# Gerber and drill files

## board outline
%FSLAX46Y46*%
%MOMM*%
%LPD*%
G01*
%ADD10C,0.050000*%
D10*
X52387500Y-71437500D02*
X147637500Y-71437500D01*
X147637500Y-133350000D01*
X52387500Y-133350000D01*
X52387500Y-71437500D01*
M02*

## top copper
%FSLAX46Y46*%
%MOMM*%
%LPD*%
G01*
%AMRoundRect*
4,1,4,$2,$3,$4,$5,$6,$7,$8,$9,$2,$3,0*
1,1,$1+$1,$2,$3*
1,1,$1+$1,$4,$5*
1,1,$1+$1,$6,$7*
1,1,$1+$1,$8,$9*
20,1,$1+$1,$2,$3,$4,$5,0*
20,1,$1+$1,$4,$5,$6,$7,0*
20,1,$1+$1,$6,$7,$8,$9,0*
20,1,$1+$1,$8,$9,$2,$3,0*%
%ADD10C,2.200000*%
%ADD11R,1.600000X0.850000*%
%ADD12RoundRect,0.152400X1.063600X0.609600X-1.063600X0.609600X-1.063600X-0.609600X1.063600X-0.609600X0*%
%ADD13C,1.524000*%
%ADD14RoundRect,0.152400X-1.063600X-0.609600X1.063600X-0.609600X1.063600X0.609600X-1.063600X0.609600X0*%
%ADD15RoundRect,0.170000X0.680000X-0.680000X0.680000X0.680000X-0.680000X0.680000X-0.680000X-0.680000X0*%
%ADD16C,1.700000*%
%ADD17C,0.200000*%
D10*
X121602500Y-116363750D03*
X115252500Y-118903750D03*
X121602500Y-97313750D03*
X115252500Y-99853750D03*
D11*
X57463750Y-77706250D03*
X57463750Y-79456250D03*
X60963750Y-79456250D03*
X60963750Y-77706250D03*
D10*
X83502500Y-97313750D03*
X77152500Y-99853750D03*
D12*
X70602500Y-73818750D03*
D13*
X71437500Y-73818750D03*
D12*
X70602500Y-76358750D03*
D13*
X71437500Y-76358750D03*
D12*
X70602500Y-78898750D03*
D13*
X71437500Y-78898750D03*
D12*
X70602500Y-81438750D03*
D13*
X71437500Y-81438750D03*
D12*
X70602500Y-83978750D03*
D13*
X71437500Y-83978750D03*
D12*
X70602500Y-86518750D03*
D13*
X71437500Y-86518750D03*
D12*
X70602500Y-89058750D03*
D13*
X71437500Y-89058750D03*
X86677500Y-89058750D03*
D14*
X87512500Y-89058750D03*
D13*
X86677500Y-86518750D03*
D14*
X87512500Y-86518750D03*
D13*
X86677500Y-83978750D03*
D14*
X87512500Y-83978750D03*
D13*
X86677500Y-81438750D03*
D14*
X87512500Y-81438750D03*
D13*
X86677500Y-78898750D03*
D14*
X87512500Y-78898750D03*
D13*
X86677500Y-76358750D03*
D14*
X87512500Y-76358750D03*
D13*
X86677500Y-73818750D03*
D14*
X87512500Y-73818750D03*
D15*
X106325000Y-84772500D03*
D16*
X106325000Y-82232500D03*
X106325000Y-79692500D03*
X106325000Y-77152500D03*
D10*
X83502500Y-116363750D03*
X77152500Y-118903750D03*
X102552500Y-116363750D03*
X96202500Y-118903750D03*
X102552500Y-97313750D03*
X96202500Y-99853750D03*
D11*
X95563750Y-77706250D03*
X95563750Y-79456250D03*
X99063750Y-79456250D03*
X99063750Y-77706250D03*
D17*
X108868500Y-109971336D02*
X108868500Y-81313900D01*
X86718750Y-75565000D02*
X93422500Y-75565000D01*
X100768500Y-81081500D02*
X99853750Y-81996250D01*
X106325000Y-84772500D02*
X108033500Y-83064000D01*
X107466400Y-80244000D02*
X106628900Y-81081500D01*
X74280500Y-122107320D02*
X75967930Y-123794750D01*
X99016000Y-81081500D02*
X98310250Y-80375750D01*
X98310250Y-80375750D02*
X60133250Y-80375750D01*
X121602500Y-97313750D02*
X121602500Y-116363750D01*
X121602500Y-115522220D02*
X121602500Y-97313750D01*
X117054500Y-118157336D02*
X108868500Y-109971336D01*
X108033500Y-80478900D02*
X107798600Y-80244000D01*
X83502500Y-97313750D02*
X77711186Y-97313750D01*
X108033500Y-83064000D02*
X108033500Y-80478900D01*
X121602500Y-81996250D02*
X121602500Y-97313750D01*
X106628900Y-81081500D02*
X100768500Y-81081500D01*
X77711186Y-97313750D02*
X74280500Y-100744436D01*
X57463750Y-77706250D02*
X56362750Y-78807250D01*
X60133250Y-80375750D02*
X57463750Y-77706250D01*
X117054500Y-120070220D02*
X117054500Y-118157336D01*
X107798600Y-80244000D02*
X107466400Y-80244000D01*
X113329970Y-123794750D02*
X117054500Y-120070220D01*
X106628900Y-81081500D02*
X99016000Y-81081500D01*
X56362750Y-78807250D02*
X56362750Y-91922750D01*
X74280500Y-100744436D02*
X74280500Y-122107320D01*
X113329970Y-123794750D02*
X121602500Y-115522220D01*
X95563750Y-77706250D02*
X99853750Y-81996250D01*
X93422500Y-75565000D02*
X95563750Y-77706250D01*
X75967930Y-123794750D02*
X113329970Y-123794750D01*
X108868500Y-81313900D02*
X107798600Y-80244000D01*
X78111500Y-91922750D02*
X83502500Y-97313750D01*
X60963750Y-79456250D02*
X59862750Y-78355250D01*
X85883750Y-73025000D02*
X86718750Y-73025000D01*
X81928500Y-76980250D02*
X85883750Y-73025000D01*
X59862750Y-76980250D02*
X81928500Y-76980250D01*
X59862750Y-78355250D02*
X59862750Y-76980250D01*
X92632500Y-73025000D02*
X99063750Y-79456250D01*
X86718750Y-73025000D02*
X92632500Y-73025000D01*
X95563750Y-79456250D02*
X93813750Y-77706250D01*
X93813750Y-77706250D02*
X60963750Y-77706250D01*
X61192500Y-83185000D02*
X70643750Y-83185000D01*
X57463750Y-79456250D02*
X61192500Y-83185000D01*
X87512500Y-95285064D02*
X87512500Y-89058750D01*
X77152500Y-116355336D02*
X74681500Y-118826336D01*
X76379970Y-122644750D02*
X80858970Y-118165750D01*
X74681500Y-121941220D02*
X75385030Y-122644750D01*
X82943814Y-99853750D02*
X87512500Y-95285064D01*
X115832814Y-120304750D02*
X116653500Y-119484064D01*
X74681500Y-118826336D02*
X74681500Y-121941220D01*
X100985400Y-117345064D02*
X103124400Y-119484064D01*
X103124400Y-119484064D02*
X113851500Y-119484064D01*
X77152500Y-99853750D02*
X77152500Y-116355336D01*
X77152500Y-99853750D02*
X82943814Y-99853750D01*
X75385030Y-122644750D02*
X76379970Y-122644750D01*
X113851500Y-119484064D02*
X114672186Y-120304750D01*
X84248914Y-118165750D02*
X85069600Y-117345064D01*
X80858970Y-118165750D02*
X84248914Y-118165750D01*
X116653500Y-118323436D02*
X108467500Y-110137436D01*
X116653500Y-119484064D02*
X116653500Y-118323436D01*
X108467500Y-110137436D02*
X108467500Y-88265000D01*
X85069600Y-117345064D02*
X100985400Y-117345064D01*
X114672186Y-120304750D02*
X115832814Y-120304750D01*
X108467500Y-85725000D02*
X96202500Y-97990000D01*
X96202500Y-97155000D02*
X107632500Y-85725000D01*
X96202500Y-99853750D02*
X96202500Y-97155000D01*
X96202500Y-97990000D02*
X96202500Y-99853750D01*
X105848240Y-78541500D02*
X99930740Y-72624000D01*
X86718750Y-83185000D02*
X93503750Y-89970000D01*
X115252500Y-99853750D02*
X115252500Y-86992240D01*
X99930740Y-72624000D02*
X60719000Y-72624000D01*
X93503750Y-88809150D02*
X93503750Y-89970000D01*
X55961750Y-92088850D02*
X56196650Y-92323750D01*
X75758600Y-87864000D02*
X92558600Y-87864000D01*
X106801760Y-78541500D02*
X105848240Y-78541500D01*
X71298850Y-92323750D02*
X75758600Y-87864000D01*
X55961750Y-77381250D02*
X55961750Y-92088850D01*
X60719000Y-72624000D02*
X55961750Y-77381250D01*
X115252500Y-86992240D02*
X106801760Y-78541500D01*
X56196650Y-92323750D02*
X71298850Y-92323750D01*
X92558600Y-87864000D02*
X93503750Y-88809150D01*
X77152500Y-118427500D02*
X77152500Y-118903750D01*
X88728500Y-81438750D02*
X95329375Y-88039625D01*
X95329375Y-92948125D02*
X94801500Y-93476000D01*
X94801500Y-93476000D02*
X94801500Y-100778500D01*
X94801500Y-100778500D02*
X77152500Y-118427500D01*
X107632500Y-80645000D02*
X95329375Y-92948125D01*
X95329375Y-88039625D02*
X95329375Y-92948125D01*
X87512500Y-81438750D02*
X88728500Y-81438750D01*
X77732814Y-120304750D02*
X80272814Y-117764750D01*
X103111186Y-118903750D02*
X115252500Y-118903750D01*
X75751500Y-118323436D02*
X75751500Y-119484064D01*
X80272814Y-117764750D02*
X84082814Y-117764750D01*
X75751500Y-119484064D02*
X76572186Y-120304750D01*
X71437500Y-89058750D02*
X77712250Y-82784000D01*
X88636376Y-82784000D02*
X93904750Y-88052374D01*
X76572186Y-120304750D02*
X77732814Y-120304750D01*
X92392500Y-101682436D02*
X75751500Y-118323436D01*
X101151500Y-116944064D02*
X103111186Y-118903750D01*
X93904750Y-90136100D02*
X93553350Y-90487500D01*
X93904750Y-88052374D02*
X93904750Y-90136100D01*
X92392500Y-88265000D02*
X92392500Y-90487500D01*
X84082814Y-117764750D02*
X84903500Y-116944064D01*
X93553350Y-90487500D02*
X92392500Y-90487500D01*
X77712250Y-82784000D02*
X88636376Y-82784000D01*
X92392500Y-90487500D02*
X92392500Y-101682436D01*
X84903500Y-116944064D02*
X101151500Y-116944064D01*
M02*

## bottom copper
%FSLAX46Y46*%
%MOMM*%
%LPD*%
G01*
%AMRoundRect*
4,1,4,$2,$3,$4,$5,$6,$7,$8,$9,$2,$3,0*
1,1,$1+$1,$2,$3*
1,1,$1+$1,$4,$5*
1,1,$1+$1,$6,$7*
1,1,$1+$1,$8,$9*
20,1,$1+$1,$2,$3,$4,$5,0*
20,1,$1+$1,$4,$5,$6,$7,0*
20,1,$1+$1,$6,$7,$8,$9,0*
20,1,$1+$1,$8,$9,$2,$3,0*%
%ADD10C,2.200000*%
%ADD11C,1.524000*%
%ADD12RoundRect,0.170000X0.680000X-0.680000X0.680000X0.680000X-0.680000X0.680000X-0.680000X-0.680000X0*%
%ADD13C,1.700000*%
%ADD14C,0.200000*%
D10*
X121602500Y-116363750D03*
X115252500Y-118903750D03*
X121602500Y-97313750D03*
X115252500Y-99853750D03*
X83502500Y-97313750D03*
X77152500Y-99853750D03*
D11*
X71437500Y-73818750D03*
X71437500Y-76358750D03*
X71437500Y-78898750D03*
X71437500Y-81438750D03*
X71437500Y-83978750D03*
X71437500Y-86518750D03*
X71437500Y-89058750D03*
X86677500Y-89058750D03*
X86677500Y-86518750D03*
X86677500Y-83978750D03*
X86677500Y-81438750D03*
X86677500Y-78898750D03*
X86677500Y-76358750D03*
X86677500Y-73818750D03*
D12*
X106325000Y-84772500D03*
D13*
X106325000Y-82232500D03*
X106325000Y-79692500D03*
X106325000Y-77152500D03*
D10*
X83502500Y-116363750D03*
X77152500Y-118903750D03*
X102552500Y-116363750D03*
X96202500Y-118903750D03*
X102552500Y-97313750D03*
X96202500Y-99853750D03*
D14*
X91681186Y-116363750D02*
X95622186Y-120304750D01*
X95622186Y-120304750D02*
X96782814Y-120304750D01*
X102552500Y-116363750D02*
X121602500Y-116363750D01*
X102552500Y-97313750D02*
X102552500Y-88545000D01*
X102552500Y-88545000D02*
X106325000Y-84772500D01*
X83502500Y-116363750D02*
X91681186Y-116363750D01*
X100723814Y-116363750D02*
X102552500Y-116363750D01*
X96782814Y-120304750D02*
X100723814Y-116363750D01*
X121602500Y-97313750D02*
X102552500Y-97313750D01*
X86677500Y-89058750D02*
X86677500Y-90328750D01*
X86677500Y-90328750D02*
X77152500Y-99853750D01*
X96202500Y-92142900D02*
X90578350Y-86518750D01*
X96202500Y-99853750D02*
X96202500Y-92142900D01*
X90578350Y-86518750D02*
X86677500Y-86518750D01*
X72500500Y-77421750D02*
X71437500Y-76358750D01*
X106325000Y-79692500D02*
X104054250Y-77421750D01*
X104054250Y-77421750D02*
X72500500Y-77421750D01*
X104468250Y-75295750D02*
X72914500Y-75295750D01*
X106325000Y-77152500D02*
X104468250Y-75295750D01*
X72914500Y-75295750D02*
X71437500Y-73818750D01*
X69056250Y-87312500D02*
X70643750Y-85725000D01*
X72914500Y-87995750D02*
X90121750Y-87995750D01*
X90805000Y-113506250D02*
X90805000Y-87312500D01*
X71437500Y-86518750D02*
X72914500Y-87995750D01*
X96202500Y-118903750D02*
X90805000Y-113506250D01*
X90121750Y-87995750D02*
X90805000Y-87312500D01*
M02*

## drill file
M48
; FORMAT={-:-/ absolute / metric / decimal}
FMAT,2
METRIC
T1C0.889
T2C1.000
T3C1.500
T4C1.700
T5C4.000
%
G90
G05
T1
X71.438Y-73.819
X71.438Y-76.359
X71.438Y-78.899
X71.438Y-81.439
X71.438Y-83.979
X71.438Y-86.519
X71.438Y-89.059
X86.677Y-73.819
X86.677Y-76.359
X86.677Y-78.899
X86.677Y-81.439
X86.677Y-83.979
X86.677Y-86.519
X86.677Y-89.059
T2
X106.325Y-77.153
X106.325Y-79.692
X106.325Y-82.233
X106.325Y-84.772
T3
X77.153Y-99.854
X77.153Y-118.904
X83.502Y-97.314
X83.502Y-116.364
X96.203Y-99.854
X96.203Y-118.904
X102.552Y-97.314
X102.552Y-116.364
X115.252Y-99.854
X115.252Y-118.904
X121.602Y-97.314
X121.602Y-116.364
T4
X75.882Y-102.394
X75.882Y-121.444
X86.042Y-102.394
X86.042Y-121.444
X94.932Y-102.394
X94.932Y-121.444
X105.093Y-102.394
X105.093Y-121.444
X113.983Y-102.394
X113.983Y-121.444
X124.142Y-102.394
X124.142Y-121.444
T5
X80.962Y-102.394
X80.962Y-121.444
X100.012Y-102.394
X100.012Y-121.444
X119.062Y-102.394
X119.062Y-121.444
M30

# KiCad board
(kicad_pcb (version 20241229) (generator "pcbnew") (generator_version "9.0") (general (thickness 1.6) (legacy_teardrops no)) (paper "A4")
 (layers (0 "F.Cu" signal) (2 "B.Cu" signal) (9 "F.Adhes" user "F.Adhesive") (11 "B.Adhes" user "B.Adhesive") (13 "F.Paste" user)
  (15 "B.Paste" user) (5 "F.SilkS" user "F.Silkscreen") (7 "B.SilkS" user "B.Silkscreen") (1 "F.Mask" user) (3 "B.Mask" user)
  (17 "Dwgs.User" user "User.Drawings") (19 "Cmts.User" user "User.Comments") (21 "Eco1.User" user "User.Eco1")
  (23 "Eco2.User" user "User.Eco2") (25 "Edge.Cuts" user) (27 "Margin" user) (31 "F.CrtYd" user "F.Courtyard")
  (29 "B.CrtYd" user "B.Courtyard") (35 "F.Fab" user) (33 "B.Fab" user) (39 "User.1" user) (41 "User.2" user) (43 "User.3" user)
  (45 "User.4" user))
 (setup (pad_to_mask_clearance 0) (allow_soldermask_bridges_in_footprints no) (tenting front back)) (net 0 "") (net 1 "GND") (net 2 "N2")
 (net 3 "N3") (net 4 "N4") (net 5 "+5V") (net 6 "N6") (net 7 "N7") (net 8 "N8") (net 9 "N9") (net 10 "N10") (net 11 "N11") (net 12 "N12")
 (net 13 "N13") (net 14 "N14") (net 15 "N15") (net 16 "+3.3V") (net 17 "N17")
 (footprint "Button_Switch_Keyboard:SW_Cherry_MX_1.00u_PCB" (layer "F.Cu") (at 121.6025 116.36375)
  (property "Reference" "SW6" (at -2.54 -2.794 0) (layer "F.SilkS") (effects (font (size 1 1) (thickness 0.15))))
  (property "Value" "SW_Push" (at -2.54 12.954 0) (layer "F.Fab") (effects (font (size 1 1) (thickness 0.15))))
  (pad "" np_thru_hole circle (at -7.62 5.08) (size 1.7 1.7) (drill 1.7) (layers "*.Cu" "*.Mask"))
  (pad "" np_thru_hole circle (at -2.54 5.08) (size 4 4) (drill 4) (layers "*.Cu" "*.Mask"))
  (pad "" np_thru_hole circle (at 2.54 5.08) (size 1.7 1.7) (drill 1.7) (layers "*.Cu" "*.Mask"))
  (pad "1" thru_hole circle (at 0 0) (size 2.2 2.2) (drill 1.5) (layers "*.Cu" "*.Mask") (remove_unused_layers no) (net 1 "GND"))
  (pad "2" thru_hole circle (at -6.35 2.54) (size 2.2 2.2) (drill 1.5) (layers "*.Cu" "*.Mask") (remove_unused_layers no) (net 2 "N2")))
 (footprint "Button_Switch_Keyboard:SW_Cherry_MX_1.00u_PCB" (layer "F.Cu") (at 121.6025 97.31375)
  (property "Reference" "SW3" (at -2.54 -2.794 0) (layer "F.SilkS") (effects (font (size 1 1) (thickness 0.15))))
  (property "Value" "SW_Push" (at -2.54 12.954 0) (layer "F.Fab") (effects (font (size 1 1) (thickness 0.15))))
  (pad "" np_thru_hole circle (at -7.62 5.08) (size 1.7 1.7) (drill 1.7) (layers "*.Cu" "*.Mask"))
  (pad "" np_thru_hole circle (at -2.54 5.08) (size 4 4) (drill 4) (layers "*.Cu" "*.Mask"))
  (pad "" np_thru_hole circle (at 2.54 5.08) (size 1.7 1.7) (drill 1.7) (layers "*.Cu" "*.Mask"))
  (pad "1" thru_hole circle (at 0 0) (size 2.2 2.2) (drill 1.5) (layers "*.Cu" "*.Mask") (remove_unused_layers no) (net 1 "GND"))
  (pad "2" thru_hole circle (at -6.35 2.54) (size 2.2 2.2) (drill 1.5) (layers "*.Cu" "*.Mask") (remove_unused_layers no) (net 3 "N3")))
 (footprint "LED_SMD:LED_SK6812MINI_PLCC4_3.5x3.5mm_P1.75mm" (layer "F.Cu") (at 59.21375 78.58125)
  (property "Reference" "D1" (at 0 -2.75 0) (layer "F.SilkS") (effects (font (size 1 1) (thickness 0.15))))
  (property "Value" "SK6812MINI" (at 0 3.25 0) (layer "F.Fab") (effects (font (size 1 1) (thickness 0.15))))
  (pad "1" smd rect (at -1.75 -0.875) (size 1.6 0.85) (layers "F.Cu" "F.Mask" "F.Paste") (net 1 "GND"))
  (pad "2" smd rect (at -1.75 0.875) (size 1.6 0.85) (layers "F.Cu" "F.Mask" "F.Paste") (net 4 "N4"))
  (pad "3" smd rect (at 1.75 0.875) (size 1.6 0.85) (layers "F.Cu" "F.Mask" "F.Paste") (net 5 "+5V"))
  (pad "4" smd rect (at 1.75 -0.875) (size 1.6 0.85) (layers "F.Cu" "F.Mask" "F.Paste") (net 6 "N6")))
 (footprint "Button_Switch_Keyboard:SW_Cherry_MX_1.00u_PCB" (layer "F.Cu") (at 83.5025 97.31375)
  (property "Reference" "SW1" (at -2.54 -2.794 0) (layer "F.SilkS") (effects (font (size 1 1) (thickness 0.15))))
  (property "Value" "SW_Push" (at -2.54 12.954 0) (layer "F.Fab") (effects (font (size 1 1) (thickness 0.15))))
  (pad "" np_thru_hole circle (at -7.62 5.08) (size 1.7 1.7) (drill 1.7) (layers "*.Cu" "*.Mask"))
  (pad "" np_thru_hole circle (at -2.54 5.08) (size 4 4) (drill 4) (layers "*.Cu" "*.Mask"))
  (pad "" np_thru_hole circle (at 2.54 5.08) (size 1.7 1.7) (drill 1.7) (layers "*.Cu" "*.Mask"))
  (pad "1" thru_hole circle (at 0 0) (size 2.2 2.2) (drill 1.5) (layers "*.Cu" "*.Mask") (remove_unused_layers no) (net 1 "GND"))
  (pad "2" thru_hole circle (at -6.35 2.54) (size 2.2 2.2) (drill 1.5) (layers "*.Cu" "*.Mask") (remove_unused_layers no) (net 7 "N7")))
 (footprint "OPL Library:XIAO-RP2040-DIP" (layer "F.Cu") (at 79.0575 81.43875)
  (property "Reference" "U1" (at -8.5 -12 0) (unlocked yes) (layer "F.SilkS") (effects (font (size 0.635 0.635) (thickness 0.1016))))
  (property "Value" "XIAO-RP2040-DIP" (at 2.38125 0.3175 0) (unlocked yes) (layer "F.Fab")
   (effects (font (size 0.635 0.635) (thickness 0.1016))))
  (pad "1" smd roundrect (at -8.455 -7.62 180) (size 2.432 1.524) (layers "F.Cu" "F.Mask") (roundrect_rratio 0.1) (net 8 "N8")
   (thermal_bridge_angle 45))
  (pad "1" thru_hole circle (at -7.62 -7.62 180) (size 1.524 1.524) (drill 0.889) (layers "*.Cu" "*.Mask") (remove_unused_layers no)
   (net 8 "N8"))
  (pad "2" smd roundrect (at -8.455 -5.08 180) (size 2.432 1.524) (layers "F.Cu" "F.Mask") (roundrect_rratio 0.1) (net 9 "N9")
   (thermal_bridge_angle 45))
  (pad "2" thru_hole circle (at -7.62 -5.08 180) (size 1.524 1.524) (drill 0.889) (layers "*.Cu" "*.Mask") (remove_unused_layers no)
   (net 9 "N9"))
  (pad "3" smd roundrect (at -8.455 -2.54 180) (size 2.432 1.524) (layers "F.Cu" "F.Mask") (roundrect_rratio 0.1) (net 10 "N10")
   (thermal_bridge_angle 45))
  (pad "3" thru_hole circle (at -7.62 -2.54 180) (size 1.524 1.524) (drill 0.889) (layers "*.Cu" "*.Mask") (remove_unused_layers no)
   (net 10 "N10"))
  (pad "4" smd roundrect (at -8.455 0 180) (size 2.432 1.524) (layers "F.Cu" "F.Mask") (roundrect_rratio 0.1) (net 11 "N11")
   (thermal_bridge_angle 45))
  (pad "4" thru_hole circle (at -7.62 0 180) (size 1.524 1.524) (drill 0.889) (layers "*.Cu" "*.Mask") (remove_unused_layers no)
   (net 11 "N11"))
  (pad "5" smd roundrect (at -8.455 2.54 180) (size 2.432 1.524) (layers "F.Cu" "F.Mask") (roundrect_rratio 0.1) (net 4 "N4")
   (thermal_bridge_angle 45))
  (pad "5" thru_hole circle (at -7.62 2.54 180) (size 1.524 1.524) (drill 0.889) (layers "*.Cu" "*.Mask") (remove_unused_layers no)
   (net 4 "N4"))
  (pad "6" smd roundrect (at -8.455 5.08 180) (size 2.432 1.524) (layers "F.Cu" "F.Mask") (roundrect_rratio 0.1) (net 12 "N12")
   (thermal_bridge_angle 45))
  (pad "6" thru_hole circle (at -7.62 5.08 180) (size 1.524 1.524) (drill 0.889) (layers "*.Cu" "*.Mask") (remove_unused_layers no)
   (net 12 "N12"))
  (pad "7" smd roundrect (at -8.455 7.62 180) (size 2.432 1.524) (layers "F.Cu" "F.Mask") (roundrect_rratio 0.1) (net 2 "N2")
   (thermal_bridge_angle 45))
  (pad "7" thru_hole circle (at -7.62 7.62 180) (size 1.524 1.524) (drill 0.889) (layers "*.Cu" "*.Mask") (remove_unused_layers no)
   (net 2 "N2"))
  (pad "8" thru_hole circle (at 7.62 7.62) (size 1.524 1.524) (drill 0.889) (layers "*.Cu" "*.Mask") (remove_unused_layers no) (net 7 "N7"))
  (pad "8" smd roundrect (at 8.455 7.62) (size 2.432 1.524) (layers "F.Cu" "F.Mask") (roundrect_rratio 0.1) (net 7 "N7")
   (thermal_bridge_angle 45))
  (pad "9" thru_hole circle (at 7.62 5.08) (size 1.524 1.524) (drill 0.889) (layers "*.Cu" "*.Mask") (remove_unused_layers no)
   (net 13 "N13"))
  (pad "9" smd roundrect (at 8.455 5.08) (size 2.432 1.524) (layers "F.Cu" "F.Mask") (roundrect_rratio 0.1) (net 13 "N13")
   (thermal_bridge_angle 45))
  (pad "10" thru_hole circle (at 7.62 2.54) (size 1.524 1.524) (drill 0.889) (layers "*.Cu" "*.Mask") (remove_unused_layers no) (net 3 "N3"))
  (pad "10" smd roundrect (at 8.455 2.54) (size 2.432 1.524) (layers "F.Cu" "F.Mask") (roundrect_rratio 0.1) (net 3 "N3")
   (thermal_bridge_angle 45))
  (pad "11" thru_hole circle (at 7.62 0) (size 1.524 1.524) (drill 0.889) (layers "*.Cu" "*.Mask") (remove_unused_layers no) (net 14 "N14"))
  (pad "11" smd roundrect (at 8.455 0) (size 2.432 1.524) (layers "F.Cu" "F.Mask") (roundrect_rratio 0.1) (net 14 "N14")
   (thermal_bridge_angle 45))
  (pad "12" thru_hole circle (at 7.62 -2.54) (size 1.524 1.524) (drill 0.889) (layers "*.Cu" "*.Mask") (remove_unused_layers no)
   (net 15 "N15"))
  (pad "12" smd roundrect (at 8.455 -2.54) (size 2.432 1.524) (layers "F.Cu" "F.Mask") (roundrect_rratio 0.1) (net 15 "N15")
   (thermal_bridge_angle 45))
  (pad "13" thru_hole circle (at 7.62 -5.08) (size 1.524 1.524) (drill 0.889) (layers "*.Cu" "*.Mask") (remove_unused_layers no)
   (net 1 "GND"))
  (pad "13" smd roundrect (at 8.455 -5.08) (size 2.432 1.524) (layers "F.Cu" "F.Mask") (roundrect_rratio 0.1) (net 1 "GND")
   (thermal_bridge_angle 45))
  (pad "14" thru_hole circle (at 7.62 -7.62) (size 1.524 1.524) (drill 0.889) (layers "*.Cu" "*.Mask") (remove_unused_layers no)
   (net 5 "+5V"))
  (pad "14" smd roundrect (at 8.455 -7.62) (size 2.432 1.524) (layers "F.Cu" "F.Mask") (roundrect_rratio 0.1) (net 5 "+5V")
   (thermal_bridge_angle 45)))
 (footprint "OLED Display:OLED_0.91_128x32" (layer "F.Cu") (at 106.325 84.7725 90)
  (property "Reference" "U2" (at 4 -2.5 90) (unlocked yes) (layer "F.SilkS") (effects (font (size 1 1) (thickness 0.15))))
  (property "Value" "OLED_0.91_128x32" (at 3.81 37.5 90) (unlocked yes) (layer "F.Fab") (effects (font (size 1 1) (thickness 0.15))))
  (pad "1" thru_hole roundrect (at 0 0 90) (size 1.7 1.7) (drill 1) (layers "*.Cu" "*.Mask") (remove_unused_layers no)
   (roundrect_rratio 0.1) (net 1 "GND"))
  (pad "2" thru_hole circle (at 2.54 0 90) (size 1.7 1.7) (drill 1) (layers "*.Cu" "*.Mask") (remove_unused_layers no) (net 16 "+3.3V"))
  (pad "3" thru_hole circle (at 5.08 0 90) (size 1.7 1.7) (drill 1) (layers "*.Cu" "*.Mask") (remove_unused_layers no) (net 9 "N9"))
  (pad "4" thru_hole circle (at 7.62 0 90) (size 1.7 1.7) (drill 1) (layers "*.Cu" "*.Mask") (remove_unused_layers no) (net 8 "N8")))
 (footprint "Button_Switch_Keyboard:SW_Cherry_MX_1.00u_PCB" (layer "F.Cu") (at 83.5025 116.36375)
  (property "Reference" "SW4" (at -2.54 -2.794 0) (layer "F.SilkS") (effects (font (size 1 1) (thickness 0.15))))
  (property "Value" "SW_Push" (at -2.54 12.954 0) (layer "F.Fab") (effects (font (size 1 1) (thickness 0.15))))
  (pad "" np_thru_hole circle (at -7.62 5.08) (size 1.7 1.7) (drill 1.7) (layers "*.Cu" "*.Mask"))
  (pad "" np_thru_hole circle (at -2.54 5.08) (size 4 4) (drill 4) (layers "*.Cu" "*.Mask"))
  (pad "" np_thru_hole circle (at 2.54 5.08) (size 1.7 1.7) (drill 1.7) (layers "*.Cu" "*.Mask"))
  (pad "1" thru_hole circle (at 0 0) (size 2.2 2.2) (drill 1.5) (layers "*.Cu" "*.Mask") (remove_unused_layers no) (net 1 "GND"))
  (pad "2" thru_hole circle (at -6.35 2.54) (size 2.2 2.2) (drill 1.5) (layers "*.Cu" "*.Mask") (remove_unused_layers no) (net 14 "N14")))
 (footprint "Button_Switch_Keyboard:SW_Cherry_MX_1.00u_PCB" (layer "F.Cu") (at 102.5525 116.36375)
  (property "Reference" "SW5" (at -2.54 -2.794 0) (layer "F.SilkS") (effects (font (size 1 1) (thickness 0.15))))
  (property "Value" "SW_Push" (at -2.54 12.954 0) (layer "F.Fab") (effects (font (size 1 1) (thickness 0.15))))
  (pad "" np_thru_hole circle (at -7.62 5.08) (size 1.7 1.7) (drill 1.7) (layers "*.Cu" "*.Mask"))
  (pad "" np_thru_hole circle (at -2.54 5.08) (size 4 4) (drill 4) (layers "*.Cu" "*.Mask"))
  (pad "" np_thru_hole circle (at 2.54 5.08) (size 1.7 1.7) (drill 1.7) (layers "*.Cu" "*.Mask"))
  (pad "1" thru_hole circle (at 0 0) (size 2.2 2.2) (drill 1.5) (layers "*.Cu" "*.Mask") (remove_unused_layers no) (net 1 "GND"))
  (pad "2" thru_hole circle (at -6.35 2.54) (size 2.2 2.2) (drill 1.5) (layers "*.Cu" "*.Mask") (remove_unused_layers no) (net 12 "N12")))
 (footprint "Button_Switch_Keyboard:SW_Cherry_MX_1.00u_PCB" (layer "F.Cu") (at 102.5525 97.31375)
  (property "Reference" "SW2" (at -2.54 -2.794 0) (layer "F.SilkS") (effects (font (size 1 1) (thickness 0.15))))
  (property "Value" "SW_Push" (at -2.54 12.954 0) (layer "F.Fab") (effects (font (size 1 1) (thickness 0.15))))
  (pad "" np_thru_hole circle (at -7.62 5.08) (size 1.7 1.7) (drill 1.7) (layers "*.Cu" "*.Mask"))
  (pad "" np_thru_hole circle (at -2.54 5.08) (size 4 4) (drill 4) (layers "*.Cu" "*.Mask"))
  (pad "" np_thru_hole circle (at 2.54 5.08) (size 1.7 1.7) (drill 1.7) (layers "*.Cu" "*.Mask"))
  (pad "1" thru_hole circle (at 0 0) (size 2.2 2.2) (drill 1.5) (layers "*.Cu" "*.Mask") (remove_unused_layers no) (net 1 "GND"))
  (pad "2" thru_hole circle (at -6.35 2.54) (size 2.2 2.2) (drill 1.5) (layers "*.Cu" "*.Mask") (remove_unused_layers no) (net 13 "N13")))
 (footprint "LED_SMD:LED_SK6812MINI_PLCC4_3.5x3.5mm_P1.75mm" (layer "F.Cu") (at 97.31375 78.58125)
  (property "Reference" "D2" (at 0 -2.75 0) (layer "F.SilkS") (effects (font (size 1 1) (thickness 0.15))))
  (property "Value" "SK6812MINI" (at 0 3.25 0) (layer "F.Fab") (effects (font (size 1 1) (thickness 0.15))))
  (pad "1" smd rect (at -1.75 -0.875) (size 1.6 0.85) (layers "F.Cu" "F.Mask" "F.Paste") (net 1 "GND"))
  (pad "2" smd rect (at -1.75 0.875) (size 1.6 0.85) (layers "F.Cu" "F.Mask" "F.Paste") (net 6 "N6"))
  (pad "3" smd rect (at 1.75 0.875) (size 1.6 0.85) (layers "F.Cu" "F.Mask" "F.Paste") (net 5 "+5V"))
  (pad "4" smd rect (at 1.75 -0.875) (size 1.6 0.85) (layers "F.Cu" "F.Mask" "F.Paste") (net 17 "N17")))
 (gr_rect (start 52.3875 71.4375) (end 147.6375 133.35) (stroke (width 0.05) (type default)) (fill no) (layer "Edge.Cuts"))
 (segment (start 108.8685 109.971336) (end 108.8685 81.3139) (width 0.2) (layer "F.Cu") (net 1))
 (segment (start 86.71875 75.565) (end 93.4225 75.565) (width 0.2) (layer "F.Cu") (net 1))
 (segment (start 100.7685 81.0815) (end 99.85375 81.99625) (width 0.2) (layer "F.Cu") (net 1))
 (segment (start 106.325 84.7725) (end 108.0335 83.064) (width 0.2) (layer "F.Cu") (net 1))
 (segment (start 107.4664 80.244) (end 106.6289 81.0815) (width 0.2) (layer "F.Cu") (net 1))
 (segment (start 74.2805 122.10732) (end 75.96793 123.79475) (width 0.2) (layer "F.Cu") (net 1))
 (segment (start 99.016 81.0815) (end 98.31025 80.37575) (width 0.2) (layer "F.Cu") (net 1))
 (segment (start 98.31025 80.37575) (end 60.13325 80.37575) (width 0.2) (layer "F.Cu") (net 1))
 (segment (start 121.6025 97.31375) (end 121.6025 116.36375) (width 0.2) (layer "F.Cu") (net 1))
 (segment (start 121.6025 115.52222) (end 121.6025 97.31375) (width 0.2) (layer "F.Cu") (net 1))
 (segment (start 117.0545 118.157336) (end 108.8685 109.971336) (width 0.2) (layer "F.Cu") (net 1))
 (segment (start 108.0335 80.4789) (end 107.7986 80.244) (width 0.2) (layer "F.Cu") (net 1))
 (segment (start 83.5025 97.31375) (end 77.711186 97.31375) (width 0.2) (layer "F.Cu") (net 1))
 (segment (start 108.0335 83.064) (end 108.0335 80.4789) (width 0.2) (layer "F.Cu") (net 1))
 (segment (start 121.6025 81.99625) (end 121.6025 97.31375) (width 0.2) (layer "F.Cu") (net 1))
 (segment (start 106.6289 81.0815) (end 100.7685 81.0815) (width 0.2) (layer "F.Cu") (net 1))
 (segment (start 77.711186 97.31375) (end 74.2805 100.744436) (width 0.2) (layer "F.Cu") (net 1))
 (segment (start 57.46375 77.70625) (end 56.36275 78.80725) (width 0.2) (layer "F.Cu") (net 1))
 (segment (start 60.13325 80.37575) (end 57.46375 77.70625) (width 0.2) (layer "F.Cu") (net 1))
 (segment (start 117.0545 120.07022) (end 117.0545 118.157336) (width 0.2) (layer "F.Cu") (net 1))
 (segment (start 107.7986 80.244) (end 107.4664 80.244) (width 0.2) (layer "F.Cu") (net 1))
 (segment (start 113.32997 123.79475) (end 117.0545 120.07022) (width 0.2) (layer "F.Cu") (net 1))
 (segment (start 106.6289 81.0815) (end 99.016 81.0815) (width 0.2) (layer "F.Cu") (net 1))
 (segment (start 56.36275 78.80725) (end 56.36275 91.92275) (width 0.2) (layer "F.Cu") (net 1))
 (segment (start 74.2805 100.744436) (end 74.2805 122.10732) (width 0.2) (layer "F.Cu") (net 1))
 (segment (start 113.32997 123.79475) (end 121.6025 115.52222) (width 0.2) (layer "F.Cu") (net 1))
 (segment (start 95.56375 77.70625) (end 99.85375 81.99625) (width 0.2) (layer "F.Cu") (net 1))
 (segment (start 93.4225 75.565) (end 95.56375 77.70625) (width 0.2) (layer "F.Cu") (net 1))
 (segment (start 75.96793 123.79475) (end 113.32997 123.79475) (width 0.2) (layer "F.Cu") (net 1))
 (segment (start 108.8685 81.3139) (end 107.7986 80.244) (width 0.2) (layer "F.Cu") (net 1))
 (segment (start 78.1115 91.92275) (end 83.5025 97.31375) (width 0.2) (layer "F.Cu") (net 1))
 (segment (start 91.681186 116.36375) (end 95.622186 120.30475) (width 0.2) (layer "B.Cu") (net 1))
 (segment (start 95.622186 120.30475) (end 96.782814 120.30475) (width 0.2) (layer "B.Cu") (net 1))
 (segment (start 102.5525 116.36375) (end 121.6025 116.36375) (width 0.2) (layer "B.Cu") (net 1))
 (segment (start 102.5525 97.31375) (end 102.5525 88.545) (width 0.2) (layer "B.Cu") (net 1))
 (segment (start 102.5525 88.545) (end 106.325 84.7725) (width 0.2) (layer "B.Cu") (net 1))
 (segment (start 83.5025 116.36375) (end 91.681186 116.36375) (width 0.2) (layer "B.Cu") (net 1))
 (segment (start 100.723814 116.36375) (end 102.5525 116.36375) (width 0.2) (layer "B.Cu") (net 1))
 (segment (start 96.782814 120.30475) (end 100.723814 116.36375) (width 0.2) (layer "B.Cu") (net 1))
 (segment (start 121.6025 97.31375) (end 102.5525 97.31375) (width 0.2) (layer "B.Cu") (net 1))
 (segment (start 60.96375 79.45625) (end 59.86275 78.35525) (width 0.2) (layer "F.Cu") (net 5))
 (segment (start 85.88375 73.025) (end 86.71875 73.025) (width 0.2) (layer "F.Cu") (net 5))
 (segment (start 81.9285 76.98025) (end 85.88375 73.025) (width 0.2) (layer "F.Cu") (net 5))
 (segment (start 59.86275 76.98025) (end 81.9285 76.98025) (width 0.2) (layer "F.Cu") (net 5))
 (segment (start 59.86275 78.35525) (end 59.86275 76.98025) (width 0.2) (layer "F.Cu") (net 5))
 (segment (start 92.6325 73.025) (end 99.06375 79.45625) (width 0.2) (layer "F.Cu") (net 5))
 (segment (start 86.71875 73.025) (end 92.6325 73.025) (width 0.2) (layer "F.Cu") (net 5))
 (segment (start 95.56375 79.45625) (end 93.81375 77.70625) (width 0.2) (layer "F.Cu") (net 6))
 (segment (start 93.81375 77.70625) (end 60.96375 77.70625) (width 0.2) (layer "F.Cu") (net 6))
 (segment (start 61.1925 83.185) (end 70.64375 83.185) (width 0.2) (layer "F.Cu") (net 4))
 (segment (start 57.46375 79.45625) (end 61.1925 83.185) (width 0.2) (layer "F.Cu") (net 4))
 (segment (start 87.5125 95.285064) (end 87.5125 89.05875) (width 0.2) (layer "F.Cu") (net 7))
 (segment (start 77.1525 116.355336) (end 74.6815 118.826336) (width 0.2) (layer "F.Cu") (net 7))
 (segment (start 76.37997 122.64475) (end 80.85897 118.16575) (width 0.2) (layer "F.Cu") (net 7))
 (segment (start 74.6815 121.94122) (end 75.38503 122.64475) (width 0.2) (layer "F.Cu") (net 7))
 (segment (start 82.943814 99.85375) (end 87.5125 95.285064) (width 0.2) (layer "F.Cu") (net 7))
 (segment (start 115.832814 120.30475) (end 116.6535 119.484064) (width 0.2) (layer "F.Cu") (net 7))
 (segment (start 74.6815 118.826336) (end 74.6815 121.94122) (width 0.2) (layer "F.Cu") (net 7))
 (segment (start 100.9854 117.345064) (end 103.1244 119.484064) (width 0.2) (layer "F.Cu") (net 7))
 (segment (start 103.1244 119.484064) (end 113.8515 119.484064) (width 0.2) (layer "F.Cu") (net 7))
 (segment (start 77.1525 99.85375) (end 77.1525 116.355336) (width 0.2) (layer "F.Cu") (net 7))
 (segment (start 77.1525 99.85375) (end 82.943814 99.85375) (width 0.2) (layer "F.Cu") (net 7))
 (segment (start 75.38503 122.64475) (end 76.37997 122.64475) (width 0.2) (layer "F.Cu") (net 7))
 (segment (start 113.8515 119.484064) (end 114.672186 120.30475) (width 0.2) (layer "F.Cu") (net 7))
 (segment (start 84.248914 118.16575) (end 85.0696 117.345064) (width 0.2) (layer "F.Cu") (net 7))
 (segment (start 80.85897 118.16575) (end 84.248914 118.16575) (width 0.2) (layer "F.Cu") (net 7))
 (segment (start 116.6535 118.323436) (end 108.4675 110.137436) (width 0.2) (layer "F.Cu") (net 7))
 (segment (start 116.6535 119.484064) (end 116.6535 118.323436) (width 0.2) (layer "F.Cu") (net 7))
 (segment (start 108.4675 110.137436) (end 108.4675 88.265) (width 0.2) (layer "F.Cu") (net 7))
 (segment (start 85.0696 117.345064) (end 100.9854 117.345064) (width 0.2) (layer "F.Cu") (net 7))
 (segment (start 114.672186 120.30475) (end 115.832814 120.30475) (width 0.2) (layer "F.Cu") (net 7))
 (segment (start 86.6775 89.05875) (end 86.6775 90.32875) (width 0.2) (layer "B.Cu") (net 7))
 (segment (start 86.6775 90.32875) (end 77.1525 99.85375) (width 0.2) (layer "B.Cu") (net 7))
 (segment (start 108.4675 85.725) (end 96.2025 97.99) (width 0.2) (layer "F.Cu") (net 13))
 (segment (start 96.2025 97.155) (end 107.6325 85.725) (width 0.2) (layer "F.Cu") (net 13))
 (segment (start 96.2025 99.85375) (end 96.2025 97.155) (width 0.2) (layer "F.Cu") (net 13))
 (segment (start 96.2025 97.99) (end 96.2025 99.85375) (width 0.2) (layer "F.Cu") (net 13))
 (segment (start 96.2025 92.1429) (end 90.57835 86.51875) (width 0.2) (layer "B.Cu") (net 13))
 (segment (start 96.2025 99.85375) (end 96.2025 92.1429) (width 0.2) (layer "B.Cu") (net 13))
 (segment (start 90.57835 86.51875) (end 86.6775 86.51875) (width 0.2) (layer "B.Cu") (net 13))
 (segment (start 105.84824 78.5415) (end 99.93074 72.624) (width 0.2) (layer "F.Cu") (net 3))
 (segment (start 86.71875 83.185) (end 93.50375 89.97) (width 0.2) (layer "F.Cu") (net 3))
 (segment (start 115.2525 99.85375) (end 115.2525 86.99224) (width 0.2) (layer "F.Cu") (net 3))
 (segment (start 99.93074 72.624) (end 60.719 72.624) (width 0.2) (layer "F.Cu") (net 3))
 (segment (start 93.50375 88.80915) (end 93.50375 89.97) (width 0.2) (layer "F.Cu") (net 3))
 (segment (start 55.96175 92.08885) (end 56.19665 92.32375) (width 0.2) (layer "F.Cu") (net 3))
 (segment (start 75.7586 87.864) (end 92.5586 87.864) (width 0.2) (layer "F.Cu") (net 3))
 (segment (start 106.80176 78.5415) (end 105.84824 78.5415) (width 0.2) (layer "F.Cu") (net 3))
 (segment (start 71.29885 92.32375) (end 75.7586 87.864) (width 0.2) (layer "F.Cu") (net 3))
 (segment (start 55.96175 77.38125) (end 55.96175 92.08885) (width 0.2) (layer "F.Cu") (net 3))
 (segment (start 60.719 72.624) (end 55.96175 77.38125) (width 0.2) (layer "F.Cu") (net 3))
 (segment (start 115.2525 86.99224) (end 106.80176 78.5415) (width 0.2) (layer "F.Cu") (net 3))
 (segment (start 56.19665 92.32375) (end 71.29885 92.32375) (width 0.2) (layer "F.Cu") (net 3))
 (segment (start 92.5586 87.864) (end 93.50375 88.80915) (width 0.2) (layer "F.Cu") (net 3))
 (segment (start 77.1525 118.4275) (end 77.1525 118.90375) (width 0.2) (layer "F.Cu") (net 14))
 (segment (start 88.7285 81.43875) (end 95.329375 88.039625) (width 0.2) (layer "F.Cu") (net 14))
 (segment (start 95.329375 92.948125) (end 94.8015 93.476) (width 0.2) (layer "F.Cu") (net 14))
 (segment (start 94.8015 93.476) (end 94.8015 100.7785) (width 0.2) (layer "F.Cu") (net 14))
 (segment (start 94.8015 100.7785) (end 77.1525 118.4275) (width 0.2) (layer "F.Cu") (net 14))
 (segment (start 107.6325 80.645) (end 95.329375 92.948125) (width 0.2) (layer "F.Cu") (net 14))
 (segment (start 95.329375 88.039625) (end 95.329375 92.948125) (width 0.2) (layer "F.Cu") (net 14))
 (segment (start 87.5125 81.43875) (end 88.7285 81.43875) (width 0.2) (layer "F.Cu") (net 14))
 (segment (start 72.5005 77.42175) (end 71.4375 76.35875) (width 0.2) (layer "B.Cu") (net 9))
 (segment (start 106.325 79.6925) (end 104.05425 77.42175) (width 0.2) (layer "B.Cu") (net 9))
 (segment (start 104.05425 77.42175) (end 72.5005 77.42175) (width 0.2) (layer "B.Cu") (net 9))
 (segment (start 104.46825 75.29575) (end 72.9145 75.29575) (width 0.2) (layer "B.Cu") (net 8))
 (segment (start 106.325 77.1525) (end 104.46825 75.29575) (width 0.2) (layer "B.Cu") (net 8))
 (segment (start 72.9145 75.29575) (end 71.4375 73.81875) (width 0.2) (layer "B.Cu") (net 8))
 (segment (start 69.05625 87.3125) (end 70.64375 85.725) (width 0.2) (layer "B.Cu") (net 12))
 (segment (start 72.9145 87.99575) (end 90.12175 87.99575) (width 0.2) (layer "B.Cu") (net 12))
 (segment (start 90.805 113.50625) (end 90.805 87.3125) (width 0.2) (layer "B.Cu") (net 12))
 (segment (start 71.4375 86.51875) (end 72.9145 87.99575) (width 0.2) (layer "B.Cu") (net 12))
 (segment (start 96.2025 118.90375) (end 90.805 113.50625) (width 0.2) (layer "B.Cu") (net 12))
 (segment (start 90.12175 87.99575) (end 90.805 87.3125) (width 0.2) (layer "B.Cu") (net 12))
 (segment (start 77.732814 120.30475) (end 80.272814 117.76475) (width 0.2) (layer "F.Cu") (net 2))
 (segment (start 103.111186 118.90375) (end 115.2525 118.90375) (width 0.2) (layer "F.Cu") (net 2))
 (segment (start 75.7515 118.323436) (end 75.7515 119.484064) (width 0.2) (layer "F.Cu") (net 2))
 (segment (start 80.272814 117.76475) (end 84.082814 117.76475) (width 0.2) (layer "F.Cu") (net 2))
 (segment (start 75.7515 119.484064) (end 76.572186 120.30475) (width 0.2) (layer "F.Cu") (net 2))
 (segment (start 71.4375 89.05875) (end 77.71225 82.784) (width 0.2) (layer "F.Cu") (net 2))
 (segment (start 88.636376 82.784) (end 93.90475 88.052374) (width 0.2) (layer "F.Cu") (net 2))
 (segment (start 76.572186 120.30475) (end 77.732814 120.30475) (width 0.2) (layer "F.Cu") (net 2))
 (segment (start 92.3925 101.682436) (end 75.7515 118.323436) (width 0.2) (layer "F.Cu") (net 2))
 (segment (start 101.1515 116.944064) (end 103.111186 118.90375) (width 0.2) (layer "F.Cu") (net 2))
 (segment (start 93.90475 90.1361) (end 93.55335 90.4875) (width 0.2) (layer "F.Cu") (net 2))
 (segment (start 93.90475 88.052374) (end 93.90475 90.1361) (width 0.2) (layer "F.Cu") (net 2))
 (segment (start 92.3925 88.265) (end 92.3925 90.4875) (width 0.2) (layer "F.Cu") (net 2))
 (segment (start 84.082814 117.76475) (end 84.9035 116.944064) (width 0.2) (layer "F.Cu") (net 2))
 (segment (start 93.55335 90.4875) (end 92.3925 90.4875) (width 0.2) (layer "F.Cu") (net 2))
 (segment (start 77.71225 82.784) (end 88.636376 82.784) (width 0.2) (layer "F.Cu") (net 2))
 (segment (start 92.3925 90.4875) (end 92.3925 101.682436) (width 0.2) (layer "F.Cu") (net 2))
 (segment (start 84.9035 116.944064) (end 101.1515 116.944064) (width 0.2) (layer "F.Cu") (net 2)))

